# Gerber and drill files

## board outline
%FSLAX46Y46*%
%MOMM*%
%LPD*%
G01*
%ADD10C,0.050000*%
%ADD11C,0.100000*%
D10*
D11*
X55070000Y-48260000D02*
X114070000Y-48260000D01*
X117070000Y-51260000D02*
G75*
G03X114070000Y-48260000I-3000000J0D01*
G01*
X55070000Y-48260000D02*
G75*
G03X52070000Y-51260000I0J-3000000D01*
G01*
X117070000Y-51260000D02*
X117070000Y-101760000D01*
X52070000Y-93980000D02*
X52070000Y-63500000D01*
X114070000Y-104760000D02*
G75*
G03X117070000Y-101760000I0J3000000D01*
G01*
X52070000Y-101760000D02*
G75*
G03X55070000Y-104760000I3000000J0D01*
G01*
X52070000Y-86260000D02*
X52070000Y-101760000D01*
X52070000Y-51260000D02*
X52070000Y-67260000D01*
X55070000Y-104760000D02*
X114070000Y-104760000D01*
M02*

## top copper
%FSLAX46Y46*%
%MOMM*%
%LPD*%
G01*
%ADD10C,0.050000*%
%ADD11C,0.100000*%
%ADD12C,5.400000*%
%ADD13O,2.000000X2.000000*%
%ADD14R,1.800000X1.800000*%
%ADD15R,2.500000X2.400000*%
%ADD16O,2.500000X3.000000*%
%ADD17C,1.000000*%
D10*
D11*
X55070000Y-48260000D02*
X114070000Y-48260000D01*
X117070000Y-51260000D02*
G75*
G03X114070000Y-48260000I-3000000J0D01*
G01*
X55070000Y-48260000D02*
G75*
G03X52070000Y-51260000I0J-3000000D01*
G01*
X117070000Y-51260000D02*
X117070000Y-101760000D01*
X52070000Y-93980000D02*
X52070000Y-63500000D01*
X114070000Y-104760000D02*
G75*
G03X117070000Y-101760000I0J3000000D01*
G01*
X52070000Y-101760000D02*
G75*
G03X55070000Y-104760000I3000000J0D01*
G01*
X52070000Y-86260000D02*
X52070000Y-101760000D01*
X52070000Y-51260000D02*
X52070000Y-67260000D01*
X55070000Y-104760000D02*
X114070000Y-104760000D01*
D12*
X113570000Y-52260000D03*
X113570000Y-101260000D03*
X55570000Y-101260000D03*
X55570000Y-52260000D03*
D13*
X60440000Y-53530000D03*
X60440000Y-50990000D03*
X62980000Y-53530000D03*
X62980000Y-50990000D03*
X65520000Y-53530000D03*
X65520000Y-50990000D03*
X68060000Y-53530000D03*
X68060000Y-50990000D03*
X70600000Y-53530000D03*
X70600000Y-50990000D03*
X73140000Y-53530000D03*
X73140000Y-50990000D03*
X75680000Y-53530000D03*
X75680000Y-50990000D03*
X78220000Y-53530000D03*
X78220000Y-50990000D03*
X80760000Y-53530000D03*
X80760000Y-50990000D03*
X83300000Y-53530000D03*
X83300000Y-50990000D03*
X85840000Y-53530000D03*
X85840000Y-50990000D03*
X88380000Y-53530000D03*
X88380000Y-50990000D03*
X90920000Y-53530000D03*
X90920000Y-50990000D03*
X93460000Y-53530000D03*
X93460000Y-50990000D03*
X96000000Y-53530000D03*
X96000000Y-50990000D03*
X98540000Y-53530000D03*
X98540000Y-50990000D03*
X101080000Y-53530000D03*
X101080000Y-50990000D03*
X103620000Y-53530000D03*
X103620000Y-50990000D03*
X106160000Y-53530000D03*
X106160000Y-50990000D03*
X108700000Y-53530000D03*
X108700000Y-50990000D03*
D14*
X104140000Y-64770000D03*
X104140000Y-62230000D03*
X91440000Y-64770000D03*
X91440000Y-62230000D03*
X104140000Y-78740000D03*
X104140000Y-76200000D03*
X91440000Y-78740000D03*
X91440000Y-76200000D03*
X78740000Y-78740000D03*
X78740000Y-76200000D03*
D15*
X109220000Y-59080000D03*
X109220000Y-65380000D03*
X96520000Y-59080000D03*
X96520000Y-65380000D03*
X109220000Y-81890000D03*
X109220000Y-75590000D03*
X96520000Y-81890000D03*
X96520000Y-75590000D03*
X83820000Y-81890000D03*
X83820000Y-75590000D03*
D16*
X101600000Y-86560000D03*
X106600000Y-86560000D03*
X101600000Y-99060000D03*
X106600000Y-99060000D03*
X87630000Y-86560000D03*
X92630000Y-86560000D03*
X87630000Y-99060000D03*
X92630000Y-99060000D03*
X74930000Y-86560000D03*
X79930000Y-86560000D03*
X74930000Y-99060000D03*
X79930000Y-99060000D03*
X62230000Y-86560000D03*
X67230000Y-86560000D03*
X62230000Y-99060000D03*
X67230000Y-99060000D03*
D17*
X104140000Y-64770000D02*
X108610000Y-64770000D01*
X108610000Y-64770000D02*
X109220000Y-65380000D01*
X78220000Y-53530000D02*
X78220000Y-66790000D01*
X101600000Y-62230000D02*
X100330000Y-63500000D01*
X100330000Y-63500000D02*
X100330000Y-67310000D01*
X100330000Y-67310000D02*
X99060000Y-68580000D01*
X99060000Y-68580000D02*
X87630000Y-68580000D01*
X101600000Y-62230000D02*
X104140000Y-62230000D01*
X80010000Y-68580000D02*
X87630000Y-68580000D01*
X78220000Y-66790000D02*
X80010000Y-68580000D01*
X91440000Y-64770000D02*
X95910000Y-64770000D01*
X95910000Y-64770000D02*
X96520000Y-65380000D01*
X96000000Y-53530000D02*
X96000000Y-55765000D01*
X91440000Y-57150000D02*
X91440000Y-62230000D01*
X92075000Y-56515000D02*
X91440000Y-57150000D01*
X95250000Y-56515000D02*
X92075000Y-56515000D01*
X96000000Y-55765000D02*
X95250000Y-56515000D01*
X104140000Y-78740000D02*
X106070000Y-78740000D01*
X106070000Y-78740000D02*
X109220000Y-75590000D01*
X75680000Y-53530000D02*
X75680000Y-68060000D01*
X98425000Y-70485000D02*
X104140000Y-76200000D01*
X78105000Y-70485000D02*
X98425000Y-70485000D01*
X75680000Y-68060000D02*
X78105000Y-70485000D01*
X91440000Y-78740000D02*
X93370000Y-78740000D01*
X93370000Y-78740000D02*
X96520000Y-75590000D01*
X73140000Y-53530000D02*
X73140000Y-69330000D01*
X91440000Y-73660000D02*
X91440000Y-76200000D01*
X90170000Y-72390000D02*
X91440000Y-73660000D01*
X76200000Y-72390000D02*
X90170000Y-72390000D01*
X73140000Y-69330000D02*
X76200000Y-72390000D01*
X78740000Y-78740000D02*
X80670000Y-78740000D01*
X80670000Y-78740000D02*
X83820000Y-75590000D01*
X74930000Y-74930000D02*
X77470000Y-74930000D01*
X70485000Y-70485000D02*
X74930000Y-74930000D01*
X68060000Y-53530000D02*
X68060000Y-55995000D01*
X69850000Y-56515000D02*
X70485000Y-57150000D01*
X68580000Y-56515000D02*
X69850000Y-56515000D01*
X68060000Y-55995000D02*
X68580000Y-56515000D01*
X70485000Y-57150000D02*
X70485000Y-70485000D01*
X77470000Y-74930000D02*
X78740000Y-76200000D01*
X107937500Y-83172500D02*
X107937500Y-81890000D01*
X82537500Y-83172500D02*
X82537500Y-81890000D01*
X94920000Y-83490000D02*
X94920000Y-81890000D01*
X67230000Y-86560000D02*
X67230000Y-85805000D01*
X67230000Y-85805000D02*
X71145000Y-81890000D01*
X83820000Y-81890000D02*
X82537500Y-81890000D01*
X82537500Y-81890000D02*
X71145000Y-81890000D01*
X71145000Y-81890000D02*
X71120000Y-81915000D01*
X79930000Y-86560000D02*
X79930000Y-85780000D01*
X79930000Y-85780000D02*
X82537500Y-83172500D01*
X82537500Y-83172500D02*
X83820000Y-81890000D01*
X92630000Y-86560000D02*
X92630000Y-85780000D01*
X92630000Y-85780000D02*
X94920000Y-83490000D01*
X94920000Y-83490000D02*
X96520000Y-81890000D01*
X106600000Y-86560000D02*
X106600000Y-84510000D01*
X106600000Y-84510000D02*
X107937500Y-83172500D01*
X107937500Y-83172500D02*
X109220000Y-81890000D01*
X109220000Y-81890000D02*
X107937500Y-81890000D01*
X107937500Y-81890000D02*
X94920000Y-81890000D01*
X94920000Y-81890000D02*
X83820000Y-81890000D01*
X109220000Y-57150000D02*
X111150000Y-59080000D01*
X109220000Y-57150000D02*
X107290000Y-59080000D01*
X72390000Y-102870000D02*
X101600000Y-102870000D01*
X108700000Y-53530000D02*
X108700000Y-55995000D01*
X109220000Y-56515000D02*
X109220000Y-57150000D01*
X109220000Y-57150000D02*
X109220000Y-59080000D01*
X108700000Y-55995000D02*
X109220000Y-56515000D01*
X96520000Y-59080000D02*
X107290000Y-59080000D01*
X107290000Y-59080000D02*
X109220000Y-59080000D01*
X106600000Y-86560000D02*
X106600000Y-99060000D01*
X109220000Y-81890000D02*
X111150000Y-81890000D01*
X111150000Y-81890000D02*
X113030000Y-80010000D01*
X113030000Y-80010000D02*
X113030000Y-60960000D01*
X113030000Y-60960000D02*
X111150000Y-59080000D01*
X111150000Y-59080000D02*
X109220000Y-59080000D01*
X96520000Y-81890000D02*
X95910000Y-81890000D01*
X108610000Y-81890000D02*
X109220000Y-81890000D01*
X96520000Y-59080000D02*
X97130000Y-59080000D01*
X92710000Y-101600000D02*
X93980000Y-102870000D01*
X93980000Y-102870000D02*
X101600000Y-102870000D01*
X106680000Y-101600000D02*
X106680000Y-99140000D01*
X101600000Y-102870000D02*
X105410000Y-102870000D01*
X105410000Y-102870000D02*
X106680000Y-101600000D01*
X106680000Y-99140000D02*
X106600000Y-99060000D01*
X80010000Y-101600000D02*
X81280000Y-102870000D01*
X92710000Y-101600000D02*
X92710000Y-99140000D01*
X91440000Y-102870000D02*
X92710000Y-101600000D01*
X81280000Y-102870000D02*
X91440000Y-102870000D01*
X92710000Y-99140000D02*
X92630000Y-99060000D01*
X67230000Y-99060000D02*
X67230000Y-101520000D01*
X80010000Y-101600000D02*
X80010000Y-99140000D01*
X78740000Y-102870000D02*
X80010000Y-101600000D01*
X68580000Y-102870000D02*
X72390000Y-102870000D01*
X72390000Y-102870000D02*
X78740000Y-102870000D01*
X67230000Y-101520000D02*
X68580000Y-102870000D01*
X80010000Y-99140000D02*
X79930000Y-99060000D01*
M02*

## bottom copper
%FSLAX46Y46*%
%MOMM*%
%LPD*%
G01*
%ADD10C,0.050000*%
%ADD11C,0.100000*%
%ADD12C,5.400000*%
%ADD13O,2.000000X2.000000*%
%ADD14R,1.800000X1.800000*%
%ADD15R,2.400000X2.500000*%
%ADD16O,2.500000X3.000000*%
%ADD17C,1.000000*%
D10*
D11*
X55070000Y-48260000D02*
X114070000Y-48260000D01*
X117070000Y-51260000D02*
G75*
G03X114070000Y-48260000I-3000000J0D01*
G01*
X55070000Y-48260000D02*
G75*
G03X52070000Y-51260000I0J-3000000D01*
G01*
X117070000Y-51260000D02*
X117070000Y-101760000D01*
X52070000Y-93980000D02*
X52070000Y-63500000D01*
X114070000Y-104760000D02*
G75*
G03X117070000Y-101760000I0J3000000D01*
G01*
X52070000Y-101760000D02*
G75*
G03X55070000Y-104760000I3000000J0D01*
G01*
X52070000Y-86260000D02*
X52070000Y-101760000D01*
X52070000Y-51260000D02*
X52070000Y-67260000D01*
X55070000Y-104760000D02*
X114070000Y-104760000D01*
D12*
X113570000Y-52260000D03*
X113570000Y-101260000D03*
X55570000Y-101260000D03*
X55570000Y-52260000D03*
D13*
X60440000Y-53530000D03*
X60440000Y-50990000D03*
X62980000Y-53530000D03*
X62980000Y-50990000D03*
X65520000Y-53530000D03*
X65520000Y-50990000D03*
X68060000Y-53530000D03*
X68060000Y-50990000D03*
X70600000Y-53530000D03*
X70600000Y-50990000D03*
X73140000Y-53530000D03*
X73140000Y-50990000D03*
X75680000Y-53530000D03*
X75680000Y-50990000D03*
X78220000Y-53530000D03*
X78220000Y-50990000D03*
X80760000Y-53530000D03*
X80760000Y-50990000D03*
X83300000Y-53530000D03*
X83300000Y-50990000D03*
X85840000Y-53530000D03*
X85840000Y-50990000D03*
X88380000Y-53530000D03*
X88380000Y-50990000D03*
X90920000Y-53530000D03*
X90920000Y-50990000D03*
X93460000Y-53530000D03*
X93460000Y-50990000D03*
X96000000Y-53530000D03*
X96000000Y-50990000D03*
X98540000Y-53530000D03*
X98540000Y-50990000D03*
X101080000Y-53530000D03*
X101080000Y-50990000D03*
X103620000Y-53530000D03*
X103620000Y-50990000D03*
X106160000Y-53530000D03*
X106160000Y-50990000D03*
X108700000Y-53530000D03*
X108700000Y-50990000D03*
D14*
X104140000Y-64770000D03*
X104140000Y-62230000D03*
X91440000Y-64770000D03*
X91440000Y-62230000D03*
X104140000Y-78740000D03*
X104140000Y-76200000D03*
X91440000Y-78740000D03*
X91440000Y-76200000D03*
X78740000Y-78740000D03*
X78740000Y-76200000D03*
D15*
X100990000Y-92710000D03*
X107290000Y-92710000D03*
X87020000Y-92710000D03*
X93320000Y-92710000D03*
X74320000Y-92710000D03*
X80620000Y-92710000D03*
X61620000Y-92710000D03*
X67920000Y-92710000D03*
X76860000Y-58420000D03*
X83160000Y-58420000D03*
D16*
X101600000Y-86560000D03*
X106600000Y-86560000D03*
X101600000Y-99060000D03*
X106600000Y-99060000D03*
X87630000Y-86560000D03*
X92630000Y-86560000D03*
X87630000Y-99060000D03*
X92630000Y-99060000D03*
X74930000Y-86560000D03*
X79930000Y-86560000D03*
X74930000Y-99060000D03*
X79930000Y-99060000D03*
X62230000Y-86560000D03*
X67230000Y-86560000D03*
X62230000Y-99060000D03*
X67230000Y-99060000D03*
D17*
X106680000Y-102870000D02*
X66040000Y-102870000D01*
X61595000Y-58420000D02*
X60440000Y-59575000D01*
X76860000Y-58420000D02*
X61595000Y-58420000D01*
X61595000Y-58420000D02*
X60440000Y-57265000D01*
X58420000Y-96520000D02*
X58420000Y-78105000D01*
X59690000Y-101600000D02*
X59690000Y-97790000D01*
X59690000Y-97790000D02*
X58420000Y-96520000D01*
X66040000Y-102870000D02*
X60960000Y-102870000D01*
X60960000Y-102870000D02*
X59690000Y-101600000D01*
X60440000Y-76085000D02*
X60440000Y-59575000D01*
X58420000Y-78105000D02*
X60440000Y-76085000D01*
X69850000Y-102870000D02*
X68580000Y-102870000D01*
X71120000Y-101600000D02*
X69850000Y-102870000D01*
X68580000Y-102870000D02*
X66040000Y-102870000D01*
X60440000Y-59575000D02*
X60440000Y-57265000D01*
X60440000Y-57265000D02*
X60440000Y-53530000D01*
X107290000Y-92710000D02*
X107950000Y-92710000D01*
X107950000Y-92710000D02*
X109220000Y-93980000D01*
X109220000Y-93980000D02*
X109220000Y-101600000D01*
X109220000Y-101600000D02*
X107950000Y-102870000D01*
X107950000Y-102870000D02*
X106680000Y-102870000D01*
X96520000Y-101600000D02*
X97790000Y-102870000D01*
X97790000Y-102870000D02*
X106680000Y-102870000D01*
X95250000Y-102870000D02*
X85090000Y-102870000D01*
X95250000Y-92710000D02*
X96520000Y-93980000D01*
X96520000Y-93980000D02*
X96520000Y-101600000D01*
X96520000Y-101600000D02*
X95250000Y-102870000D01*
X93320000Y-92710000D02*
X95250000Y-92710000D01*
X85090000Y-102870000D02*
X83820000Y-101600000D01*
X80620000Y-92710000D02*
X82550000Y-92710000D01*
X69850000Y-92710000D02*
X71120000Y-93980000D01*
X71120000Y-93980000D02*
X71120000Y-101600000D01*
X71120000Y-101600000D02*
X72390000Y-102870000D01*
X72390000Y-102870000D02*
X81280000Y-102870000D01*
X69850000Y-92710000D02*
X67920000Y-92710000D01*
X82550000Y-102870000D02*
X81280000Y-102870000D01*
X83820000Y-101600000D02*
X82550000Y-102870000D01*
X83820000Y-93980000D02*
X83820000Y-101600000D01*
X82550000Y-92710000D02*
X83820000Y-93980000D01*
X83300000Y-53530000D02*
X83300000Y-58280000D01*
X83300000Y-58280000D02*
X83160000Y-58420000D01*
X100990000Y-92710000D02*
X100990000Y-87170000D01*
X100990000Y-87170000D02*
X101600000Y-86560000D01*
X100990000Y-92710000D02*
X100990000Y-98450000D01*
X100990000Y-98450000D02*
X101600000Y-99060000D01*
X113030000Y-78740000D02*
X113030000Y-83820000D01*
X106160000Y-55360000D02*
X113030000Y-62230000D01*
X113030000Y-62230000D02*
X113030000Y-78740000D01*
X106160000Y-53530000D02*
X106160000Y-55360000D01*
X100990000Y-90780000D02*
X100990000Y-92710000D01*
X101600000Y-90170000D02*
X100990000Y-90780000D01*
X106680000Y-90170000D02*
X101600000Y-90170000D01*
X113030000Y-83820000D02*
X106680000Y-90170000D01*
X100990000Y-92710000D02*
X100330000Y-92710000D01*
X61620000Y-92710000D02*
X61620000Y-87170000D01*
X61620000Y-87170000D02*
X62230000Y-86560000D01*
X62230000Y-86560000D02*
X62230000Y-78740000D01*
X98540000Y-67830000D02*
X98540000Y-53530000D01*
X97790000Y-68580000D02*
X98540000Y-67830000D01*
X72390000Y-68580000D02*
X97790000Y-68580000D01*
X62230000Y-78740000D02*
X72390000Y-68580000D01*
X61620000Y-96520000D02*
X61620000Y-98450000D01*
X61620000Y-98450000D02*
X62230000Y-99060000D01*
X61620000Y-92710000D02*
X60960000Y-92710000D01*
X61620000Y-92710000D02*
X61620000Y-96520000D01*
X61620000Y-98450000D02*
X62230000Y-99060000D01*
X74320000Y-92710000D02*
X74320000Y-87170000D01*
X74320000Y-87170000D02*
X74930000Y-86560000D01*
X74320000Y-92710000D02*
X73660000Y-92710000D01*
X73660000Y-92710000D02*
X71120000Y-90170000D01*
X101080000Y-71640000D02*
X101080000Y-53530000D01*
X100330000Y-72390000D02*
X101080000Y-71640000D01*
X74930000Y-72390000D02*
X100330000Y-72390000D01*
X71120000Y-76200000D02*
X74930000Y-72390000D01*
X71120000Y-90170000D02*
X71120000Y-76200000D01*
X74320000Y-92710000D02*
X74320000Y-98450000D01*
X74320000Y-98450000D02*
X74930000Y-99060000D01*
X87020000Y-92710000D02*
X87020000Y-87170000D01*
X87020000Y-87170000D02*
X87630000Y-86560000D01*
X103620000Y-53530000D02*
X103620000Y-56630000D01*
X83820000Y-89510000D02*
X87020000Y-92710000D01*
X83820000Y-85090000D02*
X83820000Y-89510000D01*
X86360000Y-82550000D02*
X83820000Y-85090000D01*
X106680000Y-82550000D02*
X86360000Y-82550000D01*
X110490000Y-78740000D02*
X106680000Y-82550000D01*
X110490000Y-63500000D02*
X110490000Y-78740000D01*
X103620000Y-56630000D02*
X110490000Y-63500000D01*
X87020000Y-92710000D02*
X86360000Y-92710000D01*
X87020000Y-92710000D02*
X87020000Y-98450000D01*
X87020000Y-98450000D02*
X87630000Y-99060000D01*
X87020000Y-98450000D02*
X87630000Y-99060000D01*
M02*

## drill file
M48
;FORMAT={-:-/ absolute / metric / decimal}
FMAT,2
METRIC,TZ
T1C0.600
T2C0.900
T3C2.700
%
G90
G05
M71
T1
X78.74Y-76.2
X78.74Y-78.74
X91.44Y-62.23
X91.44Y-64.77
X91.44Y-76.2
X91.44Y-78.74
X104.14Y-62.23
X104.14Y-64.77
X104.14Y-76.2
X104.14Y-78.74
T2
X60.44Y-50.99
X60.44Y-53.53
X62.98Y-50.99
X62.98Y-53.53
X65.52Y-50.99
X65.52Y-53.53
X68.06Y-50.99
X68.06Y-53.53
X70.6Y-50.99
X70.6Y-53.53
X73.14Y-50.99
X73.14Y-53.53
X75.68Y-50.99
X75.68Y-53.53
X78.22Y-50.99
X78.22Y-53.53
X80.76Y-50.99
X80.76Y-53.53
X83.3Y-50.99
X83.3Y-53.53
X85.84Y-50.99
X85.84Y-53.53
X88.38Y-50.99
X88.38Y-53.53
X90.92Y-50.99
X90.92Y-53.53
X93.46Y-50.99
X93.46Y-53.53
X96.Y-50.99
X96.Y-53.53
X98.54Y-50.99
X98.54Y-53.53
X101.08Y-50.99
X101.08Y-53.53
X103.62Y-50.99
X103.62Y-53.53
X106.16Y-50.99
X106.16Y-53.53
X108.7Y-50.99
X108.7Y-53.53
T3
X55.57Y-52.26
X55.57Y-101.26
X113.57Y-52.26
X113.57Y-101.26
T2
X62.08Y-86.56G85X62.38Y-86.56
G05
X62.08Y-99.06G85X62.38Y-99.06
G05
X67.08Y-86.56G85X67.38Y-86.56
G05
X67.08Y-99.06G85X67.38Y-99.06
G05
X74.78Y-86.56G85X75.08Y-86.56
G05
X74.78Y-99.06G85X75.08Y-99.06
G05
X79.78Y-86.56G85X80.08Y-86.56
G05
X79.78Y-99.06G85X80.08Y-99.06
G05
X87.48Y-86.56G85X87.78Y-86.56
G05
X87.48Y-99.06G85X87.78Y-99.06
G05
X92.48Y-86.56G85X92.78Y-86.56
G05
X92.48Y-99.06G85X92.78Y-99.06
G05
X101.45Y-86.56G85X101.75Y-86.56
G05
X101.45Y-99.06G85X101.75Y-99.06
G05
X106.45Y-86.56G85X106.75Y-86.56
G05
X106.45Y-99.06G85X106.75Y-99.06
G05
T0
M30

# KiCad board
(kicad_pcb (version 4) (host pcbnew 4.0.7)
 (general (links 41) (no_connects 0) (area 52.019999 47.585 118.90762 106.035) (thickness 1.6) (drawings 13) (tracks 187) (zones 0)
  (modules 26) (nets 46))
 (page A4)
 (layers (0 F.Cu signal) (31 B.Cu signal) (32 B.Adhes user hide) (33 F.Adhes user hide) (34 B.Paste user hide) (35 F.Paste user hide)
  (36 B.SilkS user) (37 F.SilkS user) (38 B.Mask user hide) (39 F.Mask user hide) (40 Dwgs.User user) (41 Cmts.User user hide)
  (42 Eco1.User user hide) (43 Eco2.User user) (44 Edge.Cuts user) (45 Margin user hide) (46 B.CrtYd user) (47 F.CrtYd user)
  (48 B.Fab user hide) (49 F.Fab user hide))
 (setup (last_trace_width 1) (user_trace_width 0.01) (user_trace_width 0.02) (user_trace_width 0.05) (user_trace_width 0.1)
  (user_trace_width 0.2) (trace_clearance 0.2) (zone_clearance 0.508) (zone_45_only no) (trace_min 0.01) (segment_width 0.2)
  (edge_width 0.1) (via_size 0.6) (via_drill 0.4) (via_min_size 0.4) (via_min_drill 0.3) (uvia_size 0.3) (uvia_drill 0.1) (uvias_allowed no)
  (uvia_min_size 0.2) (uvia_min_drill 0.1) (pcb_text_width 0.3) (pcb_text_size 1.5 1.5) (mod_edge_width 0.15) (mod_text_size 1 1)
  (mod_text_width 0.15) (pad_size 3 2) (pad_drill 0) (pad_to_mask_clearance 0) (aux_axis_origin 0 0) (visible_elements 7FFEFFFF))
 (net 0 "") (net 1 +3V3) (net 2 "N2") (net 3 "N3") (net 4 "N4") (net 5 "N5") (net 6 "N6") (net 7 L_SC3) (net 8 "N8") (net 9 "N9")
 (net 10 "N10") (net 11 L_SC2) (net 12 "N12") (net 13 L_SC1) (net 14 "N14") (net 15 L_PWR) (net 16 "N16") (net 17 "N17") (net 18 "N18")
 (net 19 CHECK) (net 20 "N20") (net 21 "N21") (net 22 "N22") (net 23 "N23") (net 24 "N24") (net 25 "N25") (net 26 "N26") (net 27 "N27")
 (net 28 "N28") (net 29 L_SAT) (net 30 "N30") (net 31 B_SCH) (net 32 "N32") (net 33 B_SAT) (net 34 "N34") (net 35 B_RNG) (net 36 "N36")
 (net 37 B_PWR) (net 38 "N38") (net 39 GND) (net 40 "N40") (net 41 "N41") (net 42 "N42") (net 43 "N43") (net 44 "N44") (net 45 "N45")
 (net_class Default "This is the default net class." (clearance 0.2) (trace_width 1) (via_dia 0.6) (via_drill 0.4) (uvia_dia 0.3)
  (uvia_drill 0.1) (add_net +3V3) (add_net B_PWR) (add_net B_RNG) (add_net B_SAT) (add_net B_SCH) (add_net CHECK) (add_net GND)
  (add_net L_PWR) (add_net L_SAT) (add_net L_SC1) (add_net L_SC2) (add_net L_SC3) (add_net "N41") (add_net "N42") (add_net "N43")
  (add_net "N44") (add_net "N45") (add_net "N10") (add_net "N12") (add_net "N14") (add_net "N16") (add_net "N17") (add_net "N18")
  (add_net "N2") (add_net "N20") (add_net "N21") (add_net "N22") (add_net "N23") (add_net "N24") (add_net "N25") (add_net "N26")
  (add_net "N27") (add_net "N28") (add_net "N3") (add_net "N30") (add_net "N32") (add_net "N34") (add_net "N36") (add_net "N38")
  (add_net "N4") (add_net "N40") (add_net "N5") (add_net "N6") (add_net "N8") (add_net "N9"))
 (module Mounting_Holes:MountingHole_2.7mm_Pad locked (layer F.Cu) (at 113.57 52.26)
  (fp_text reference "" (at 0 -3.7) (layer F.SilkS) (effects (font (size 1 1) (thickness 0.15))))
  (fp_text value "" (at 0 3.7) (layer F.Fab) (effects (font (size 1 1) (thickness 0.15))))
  (pad 1 thru_hole circle (at 0 0) (size 5.4 5.4) (drill 2.7) (layers *.Cu *.Mask)))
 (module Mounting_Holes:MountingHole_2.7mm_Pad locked (layer F.Cu) (at 113.57 101.26)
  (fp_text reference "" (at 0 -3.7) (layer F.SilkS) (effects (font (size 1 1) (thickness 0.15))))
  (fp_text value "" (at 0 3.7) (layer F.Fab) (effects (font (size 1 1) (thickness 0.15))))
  (pad 1 thru_hole circle (at 0 0) (size 5.4 5.4) (drill 2.7) (layers *.Cu *.Mask)))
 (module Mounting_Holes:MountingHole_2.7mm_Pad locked (layer F.Cu) (at 55.57 101.26)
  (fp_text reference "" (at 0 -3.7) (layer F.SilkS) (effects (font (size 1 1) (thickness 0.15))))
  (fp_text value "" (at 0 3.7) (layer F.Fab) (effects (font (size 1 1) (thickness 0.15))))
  (pad 1 thru_hole circle (at 0 0) (size 5.4 5.4) (drill 2.7) (layers *.Cu *.Mask)))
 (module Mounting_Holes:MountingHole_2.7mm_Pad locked (layer F.Cu) (at 55.57 52.26)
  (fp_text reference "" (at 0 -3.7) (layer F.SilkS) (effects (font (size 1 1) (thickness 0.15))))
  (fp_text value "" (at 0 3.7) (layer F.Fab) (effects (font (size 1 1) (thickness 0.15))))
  (pad 1 thru_hole circle (at 0 0) (size 5.4 5.4) (drill 2.7) (layers *.Cu *.Mask)))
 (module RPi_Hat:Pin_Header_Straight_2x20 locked (layer F.Cu) (at 84.57 52.26 90)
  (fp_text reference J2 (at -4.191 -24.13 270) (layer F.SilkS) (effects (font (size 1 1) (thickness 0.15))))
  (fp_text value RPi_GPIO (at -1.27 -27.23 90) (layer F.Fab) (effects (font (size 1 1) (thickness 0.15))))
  (pad 1 thru_hole oval (at -1.27 -24.13 90) (size 2 2) (drill 0.9) (layers *.Cu *.Mask F.SilkS) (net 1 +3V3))
  (pad 2 thru_hole oval (at 1.27 -24.13 90) (size 2 2) (drill 0.9) (layers *.Cu *.Mask F.SilkS) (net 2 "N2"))
  (pad 3 thru_hole oval (at -1.27 -21.59 90) (size 2 2) (drill 0.9) (layers *.Cu *.Mask F.SilkS) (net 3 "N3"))
  (pad 4 thru_hole oval (at 1.27 -21.59 90) (size 2 2) (drill 0.9) (layers *.Cu *.Mask F.SilkS) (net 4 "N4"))
  (pad 5 thru_hole oval (at -1.27 -19.05 90) (size 2 2) (drill 0.9) (layers *.Cu *.Mask F.SilkS) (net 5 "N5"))
  (pad 6 thru_hole oval (at 1.27 -19.05 90) (size 2 2) (drill 0.9) (layers *.Cu *.Mask F.SilkS) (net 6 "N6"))
  (pad 7 thru_hole oval (at -1.27 -16.51 90) (size 2 2) (drill 0.9) (layers *.Cu *.Mask F.SilkS) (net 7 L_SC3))
  (pad 8 thru_hole oval (at 1.27 -16.51 90) (size 2 2) (drill 0.9) (layers *.Cu *.Mask F.SilkS) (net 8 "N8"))
  (pad 9 thru_hole oval (at -1.27 -13.97 90) (size 2 2) (drill 0.9) (layers *.Cu *.Mask F.SilkS) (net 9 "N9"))
  (pad 10 thru_hole oval (at 1.27 -13.97 90) (size 2 2) (drill 0.9) (layers *.Cu *.Mask F.SilkS) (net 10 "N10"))
  (pad 11 thru_hole oval (at -1.27 -11.43 90) (size 2 2) (drill 0.9) (layers *.Cu *.Mask F.SilkS) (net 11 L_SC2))
  (pad 12 thru_hole oval (at 1.27 -11.43 90) (size 2 2) (drill 0.9) (layers *.Cu *.Mask F.SilkS) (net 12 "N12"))
  (pad 13 thru_hole oval (at -1.27 -8.89 90) (size 2 2) (drill 0.9) (layers *.Cu *.Mask F.SilkS) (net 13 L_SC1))
  (pad 14 thru_hole oval (at 1.27 -8.89 90) (size 2 2) (drill 0.9) (layers *.Cu *.Mask F.SilkS) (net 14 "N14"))
  (pad 15 thru_hole oval (at -1.27 -6.35 90) (size 2 2) (drill 0.9) (layers *.Cu *.Mask F.SilkS) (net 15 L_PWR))
  (pad 16 thru_hole oval (at 1.27 -6.35 90) (size 2 2) (drill 0.9) (layers *.Cu *.Mask F.SilkS) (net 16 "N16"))
  (pad 17 thru_hole oval (at -1.27 -3.81 90) (size 2 2) (drill 0.9) (layers *.Cu *.Mask F.SilkS) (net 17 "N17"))
  (pad 18 thru_hole oval (at 1.27 -3.81 90) (size 2 2) (drill 0.9) (layers *.Cu *.Mask F.SilkS) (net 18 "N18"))
  (pad 19 thru_hole oval (at -1.27 -1.27 90) (size 2 2) (drill 0.9) (layers *.Cu *.Mask F.SilkS) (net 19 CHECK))
  (pad 20 thru_hole oval (at 1.27 -1.27 90) (size 2 2) (drill 0.9) (layers *.Cu *.Mask F.SilkS) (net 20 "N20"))
  (pad 21 thru_hole oval (at -1.27 1.27 90) (size 2 2) (drill 0.9) (layers *.Cu *.Mask F.SilkS) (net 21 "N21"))
  (pad 22 thru_hole oval (at 1.27 1.27 90) (size 2 2) (drill 0.9) (layers *.Cu *.Mask F.SilkS) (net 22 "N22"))
  (pad 23 thru_hole oval (at -1.27 3.81 90) (size 2 2) (drill 0.9) (layers *.Cu *.Mask F.SilkS) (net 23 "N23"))
  (pad 24 thru_hole oval (at 1.27 3.81 90) (size 2 2) (drill 0.9) (layers *.Cu *.Mask F.SilkS) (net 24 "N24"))
  (pad 25 thru_hole oval (at -1.27 6.35 90) (size 2 2) (drill 0.9) (layers *.Cu *.Mask F.SilkS) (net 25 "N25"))
  (pad 26 thru_hole oval (at 1.27 6.35 90) (size 2 2) (drill 0.9) (layers *.Cu *.Mask F.SilkS) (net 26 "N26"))
  (pad 27 thru_hole oval (at -1.27 8.89 90) (size 2 2) (drill 0.9) (layers *.Cu *.Mask F.SilkS) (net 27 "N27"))
  (pad 28 thru_hole oval (at 1.27 8.89 90) (size 2 2) (drill 0.9) (layers *.Cu *.Mask F.SilkS) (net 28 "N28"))
  (pad 29 thru_hole oval (at -1.27 11.43 90) (size 2 2) (drill 0.9) (layers *.Cu *.Mask F.SilkS) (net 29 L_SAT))
  (pad 30 thru_hole oval (at 1.27 11.43 90) (size 2 2) (drill 0.9) (layers *.Cu *.Mask F.SilkS) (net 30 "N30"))
  (pad 31 thru_hole oval (at -1.27 13.97 90) (size 2 2) (drill 0.9) (layers *.Cu *.Mask F.SilkS) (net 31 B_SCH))
  (pad 32 thru_hole oval (at 1.27 13.97 90) (size 2 2) (drill 0.9) (layers *.Cu *.Mask F.SilkS) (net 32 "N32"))
  (pad 33 thru_hole oval (at -1.27 16.51 90) (size 2 2) (drill 0.9) (layers *.Cu *.Mask F.SilkS) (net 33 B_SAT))
  (pad 34 thru_hole oval (at 1.27 16.51 90) (size 2 2) (drill 0.9) (layers *.Cu *.Mask F.SilkS) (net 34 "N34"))
  (pad 35 thru_hole oval (at -1.27 19.05 90) (size 2 2) (drill 0.9) (layers *.Cu *.Mask F.SilkS) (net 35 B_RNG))
  (pad 36 thru_hole oval (at 1.27 19.05 90) (size 2 2) (drill 0.9) (layers *.Cu *.Mask F.SilkS) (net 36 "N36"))
  (pad 37 thru_hole oval (at -1.27 21.59 90) (size 2 2) (drill 0.9) (layers *.Cu *.Mask F.SilkS) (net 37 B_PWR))
  (pad 38 thru_hole oval (at 1.27 21.59 90) (size 2 2) (drill 0.9) (layers *.Cu *.Mask F.SilkS) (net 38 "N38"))
  (pad 39 thru_hole oval (at -1.27 24.13 90) (size 2 2) (drill 0.9) (layers *.Cu *.Mask F.SilkS) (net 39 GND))
  (pad 40 thru_hole oval (at 1.27 24.13 90) (size 2 2) (drill 0.9) (layers *.Cu *.Mask F.SilkS) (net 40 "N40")))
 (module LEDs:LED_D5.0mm (layer F.Cu) (at 104.14 64.77 90)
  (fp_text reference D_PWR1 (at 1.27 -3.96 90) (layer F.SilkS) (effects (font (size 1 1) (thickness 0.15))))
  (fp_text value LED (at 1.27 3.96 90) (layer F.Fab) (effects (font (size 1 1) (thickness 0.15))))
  (pad 1 thru_hole rect (at 0 0 90) (size 1.8 1.8) (drill 0.6) (layers *.Cu *.Mask) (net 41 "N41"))
  (pad 2 thru_hole rect (at 2.54 0 90) (size 1.8 1.8) (drill 0.6) (layers *.Cu *.Mask) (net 15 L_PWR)))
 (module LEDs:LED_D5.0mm (layer F.Cu) (at 91.44 64.77 90)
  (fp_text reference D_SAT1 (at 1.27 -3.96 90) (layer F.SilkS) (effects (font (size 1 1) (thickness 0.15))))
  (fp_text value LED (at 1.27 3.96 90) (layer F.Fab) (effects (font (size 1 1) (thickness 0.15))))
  (pad 1 thru_hole rect (at 0 0 90) (size 1.8 1.8) (drill 0.6) (layers *.Cu *.Mask) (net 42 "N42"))
  (pad 2 thru_hole rect (at 2.54 0 90) (size 1.8 1.8) (drill 0.6) (layers *.Cu *.Mask) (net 29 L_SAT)))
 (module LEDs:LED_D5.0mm (layer F.Cu) (at 104.14 78.74 90)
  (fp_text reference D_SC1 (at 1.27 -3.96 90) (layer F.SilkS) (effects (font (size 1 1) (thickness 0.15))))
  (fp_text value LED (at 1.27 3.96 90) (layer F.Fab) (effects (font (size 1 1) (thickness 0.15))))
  (pad 1 thru_hole rect (at 0 0 90) (size 1.8 1.8) (drill 0.6) (layers *.Cu *.Mask) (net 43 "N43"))
  (pad 2 thru_hole rect (at 2.54 0 90) (size 1.8 1.8) (drill 0.6) (layers *.Cu *.Mask) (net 13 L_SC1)))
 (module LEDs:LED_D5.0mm (layer F.Cu) (at 91.44 78.74 90)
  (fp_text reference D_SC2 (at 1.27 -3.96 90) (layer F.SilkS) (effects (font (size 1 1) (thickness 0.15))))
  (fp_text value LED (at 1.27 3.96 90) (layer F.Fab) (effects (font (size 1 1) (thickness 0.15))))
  (pad 1 thru_hole rect (at 0 0 90) (size 1.8 1.8) (drill 0.6) (layers *.Cu *.Mask) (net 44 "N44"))
  (pad 2 thru_hole rect (at 2.54 0 90) (size 1.8 1.8) (drill 0.6) (layers *.Cu *.Mask) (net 11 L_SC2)))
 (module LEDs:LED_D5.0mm (layer F.Cu) (at 78.74 78.74 90)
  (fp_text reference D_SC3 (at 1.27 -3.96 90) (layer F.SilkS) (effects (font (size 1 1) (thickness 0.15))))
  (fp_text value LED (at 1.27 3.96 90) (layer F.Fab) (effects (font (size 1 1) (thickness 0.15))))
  (pad 1 thru_hole rect (at 0 0 90) (size 1.8 1.8) (drill 0.6) (layers *.Cu *.Mask) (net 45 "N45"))
  (pad 2 thru_hole rect (at 2.54 0 90) (size 1.8 1.8) (drill 0.6) (layers *.Cu *.Mask) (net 7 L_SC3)))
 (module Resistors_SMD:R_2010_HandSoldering (layer B.Cu) (at 104.14 92.71)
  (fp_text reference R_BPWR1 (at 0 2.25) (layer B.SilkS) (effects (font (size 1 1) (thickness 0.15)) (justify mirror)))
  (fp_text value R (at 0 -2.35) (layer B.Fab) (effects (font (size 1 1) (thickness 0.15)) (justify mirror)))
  (pad 1 smd rect (at -3.15 0) (size 2.4 2.5) (layers B.Cu B.Paste B.Mask) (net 37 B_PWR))
  (pad 2 smd rect (at 3.15 0) (size 2.4 2.5) (layers B.Cu B.Paste B.Mask) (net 1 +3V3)))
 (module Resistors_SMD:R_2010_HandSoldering (layer B.Cu) (at 90.17 92.71)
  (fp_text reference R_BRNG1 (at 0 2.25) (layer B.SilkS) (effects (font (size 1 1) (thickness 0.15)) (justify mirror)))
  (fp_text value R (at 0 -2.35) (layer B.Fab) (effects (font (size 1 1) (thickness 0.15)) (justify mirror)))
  (pad 1 smd rect (at -3.15 0) (size 2.4 2.5) (layers B.Cu B.Paste B.Mask) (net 35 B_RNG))
  (pad 2 smd rect (at 3.15 0) (size 2.4 2.5) (layers B.Cu B.Paste B.Mask) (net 1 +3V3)))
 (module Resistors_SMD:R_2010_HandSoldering (layer B.Cu) (at 77.47 92.71)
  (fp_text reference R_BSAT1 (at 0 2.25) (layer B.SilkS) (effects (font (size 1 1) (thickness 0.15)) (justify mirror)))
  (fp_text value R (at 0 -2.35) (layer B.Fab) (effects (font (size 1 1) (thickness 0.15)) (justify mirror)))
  (pad 1 smd rect (at -3.15 0) (size 2.4 2.5) (layers B.Cu B.Paste B.Mask) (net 33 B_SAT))
  (pad 2 smd rect (at 3.15 0) (size 2.4 2.5) (layers B.Cu B.Paste B.Mask) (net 1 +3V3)))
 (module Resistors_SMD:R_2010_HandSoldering (layer B.Cu) (at 64.77 92.71)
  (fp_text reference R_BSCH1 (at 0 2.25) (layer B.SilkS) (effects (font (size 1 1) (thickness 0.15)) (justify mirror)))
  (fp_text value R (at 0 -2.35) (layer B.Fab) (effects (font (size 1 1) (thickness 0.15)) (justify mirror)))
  (pad 1 smd rect (at -3.15 0) (size 2.4 2.5) (layers B.Cu B.Paste B.Mask) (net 31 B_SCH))
  (pad 2 smd rect (at 3.15 0) (size 2.4 2.5) (layers B.Cu B.Paste B.Mask) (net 1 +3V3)))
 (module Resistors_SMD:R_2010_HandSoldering (layer B.Cu) (at 80.01 58.42)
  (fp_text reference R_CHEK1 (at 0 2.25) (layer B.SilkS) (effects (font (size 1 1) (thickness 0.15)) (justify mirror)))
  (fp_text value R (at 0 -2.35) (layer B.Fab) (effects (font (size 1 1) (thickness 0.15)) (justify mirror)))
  (pad 1 smd rect (at -3.15 0) (size 2.4 2.5) (layers B.Cu B.Paste B.Mask) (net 1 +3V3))
  (pad 2 smd rect (at 3.15 0) (size 2.4 2.5) (layers B.Cu B.Paste B.Mask) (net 19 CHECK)))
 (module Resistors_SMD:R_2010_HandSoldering (layer F.Cu) (at 109.22 62.23 270)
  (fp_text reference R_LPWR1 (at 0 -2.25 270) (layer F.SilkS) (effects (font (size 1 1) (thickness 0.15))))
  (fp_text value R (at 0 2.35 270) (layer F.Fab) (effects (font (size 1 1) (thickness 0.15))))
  (pad 1 smd rect (at -3.15 0 270) (size 2.4 2.5) (layers F.Cu F.Paste F.Mask) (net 39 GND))
  (pad 2 smd rect (at 3.15 0 270) (size 2.4 2.5) (layers F.Cu F.Paste F.Mask) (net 41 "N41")))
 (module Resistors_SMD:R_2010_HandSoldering (layer F.Cu) (at 96.52 62.23 270)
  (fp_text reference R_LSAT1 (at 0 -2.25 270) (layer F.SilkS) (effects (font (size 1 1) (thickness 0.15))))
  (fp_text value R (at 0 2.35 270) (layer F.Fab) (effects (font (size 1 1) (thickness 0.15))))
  (pad 1 smd rect (at -3.15 0 270) (size 2.4 2.5) (layers F.Cu F.Paste F.Mask) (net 39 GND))
  (pad 2 smd rect (at 3.15 0 270) (size 2.4 2.5) (layers F.Cu F.Paste F.Mask) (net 42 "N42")))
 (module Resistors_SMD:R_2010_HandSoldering (layer F.Cu) (at 109.22 78.74 90)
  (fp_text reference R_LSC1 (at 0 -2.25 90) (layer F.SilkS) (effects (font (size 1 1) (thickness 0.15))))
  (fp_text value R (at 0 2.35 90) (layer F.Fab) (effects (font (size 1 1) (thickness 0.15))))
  (pad 1 smd rect (at -3.15 0 90) (size 2.4 2.5) (layers F.Cu F.Paste F.Mask) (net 39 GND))
  (pad 2 smd rect (at 3.15 0 90) (size 2.4 2.5) (layers F.Cu F.Paste F.Mask) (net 43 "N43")))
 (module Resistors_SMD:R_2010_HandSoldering (layer F.Cu) (at 96.52 78.74 90)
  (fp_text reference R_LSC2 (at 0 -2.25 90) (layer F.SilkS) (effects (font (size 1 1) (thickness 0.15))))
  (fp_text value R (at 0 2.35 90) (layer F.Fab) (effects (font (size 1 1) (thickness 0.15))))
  (pad 1 smd rect (at -3.15 0 90) (size 2.4 2.5) (layers F.Cu F.Paste F.Mask) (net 39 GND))
  (pad 2 smd rect (at 3.15 0 90) (size 2.4 2.5) (layers F.Cu F.Paste F.Mask) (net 44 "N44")))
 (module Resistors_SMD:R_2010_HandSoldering (layer F.Cu) (at 83.82 78.74 90)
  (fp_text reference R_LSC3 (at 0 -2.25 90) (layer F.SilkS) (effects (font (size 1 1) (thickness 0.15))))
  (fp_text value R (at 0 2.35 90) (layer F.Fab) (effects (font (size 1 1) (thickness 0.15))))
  (pad 1 smd rect (at -3.15 0 90) (size 2.4 2.5) (layers F.Cu F.Paste F.Mask) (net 39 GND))
  (pad 2 smd rect (at 3.15 0 90) (size 2.4 2.5) (layers F.Cu F.Paste F.Mask) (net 45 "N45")))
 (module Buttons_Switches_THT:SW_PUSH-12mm (layer F.Cu) (at 101.6 99.06 90)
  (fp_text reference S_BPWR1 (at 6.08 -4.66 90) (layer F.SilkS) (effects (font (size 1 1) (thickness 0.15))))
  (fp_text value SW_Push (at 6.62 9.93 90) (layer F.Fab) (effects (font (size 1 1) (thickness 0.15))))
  (pad 1 thru_hole oval (at 12.5 0 90) (size 3 2.5) (drill oval 0.9 1.2) (layers *.Cu *.Mask) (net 37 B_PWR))
  (pad 2 thru_hole oval (at 12.5 5 90) (size 3 2.5) (drill oval 0.9 1.2) (layers *.Cu *.Mask) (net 39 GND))
  (pad 1 thru_hole oval (at 0 0 90) (size 3 2.5) (drill oval 0.9 1.2) (layers *.Cu *.Mask) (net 37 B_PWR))
  (pad 2 thru_hole oval (at 0 5 90) (size 3 2.5) (drill oval 0.9 1.2) (layers *.Cu *.Mask) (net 39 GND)))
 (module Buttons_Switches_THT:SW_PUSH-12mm (layer F.Cu) (at 87.63 99.06 90)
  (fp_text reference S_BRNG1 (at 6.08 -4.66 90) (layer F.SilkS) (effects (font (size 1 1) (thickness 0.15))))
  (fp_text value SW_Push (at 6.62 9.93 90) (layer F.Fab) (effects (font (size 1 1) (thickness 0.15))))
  (pad 1 thru_hole oval (at 12.5 0 90) (size 3 2.5) (drill oval 0.9 1.2) (layers *.Cu *.Mask) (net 35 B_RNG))
  (pad 2 thru_hole oval (at 12.5 5 90) (size 3 2.5) (drill oval 0.9 1.2) (layers *.Cu *.Mask) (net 39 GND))
  (pad 1 thru_hole oval (at 0 0 90) (size 3 2.5) (drill oval 0.9 1.2) (layers *.Cu *.Mask) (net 35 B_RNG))
  (pad 2 thru_hole oval (at 0 5 90) (size 3 2.5) (drill oval 0.9 1.2) (layers *.Cu *.Mask) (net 39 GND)))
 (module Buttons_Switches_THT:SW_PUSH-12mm (layer F.Cu) (at 74.93 99.06 90)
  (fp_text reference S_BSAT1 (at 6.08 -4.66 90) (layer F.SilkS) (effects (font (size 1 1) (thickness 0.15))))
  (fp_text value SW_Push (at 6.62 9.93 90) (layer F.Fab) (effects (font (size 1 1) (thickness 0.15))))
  (pad 1 thru_hole oval (at 12.5 0 90) (size 3 2.5) (drill oval 0.9 1.2) (layers *.Cu *.Mask) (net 33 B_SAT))
  (pad 2 thru_hole oval (at 12.5 5 90) (size 3 2.5) (drill oval 0.9 1.2) (layers *.Cu *.Mask) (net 39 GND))
  (pad 1 thru_hole oval (at 0 0 90) (size 3 2.5) (drill oval 0.9 1.2) (layers *.Cu *.Mask) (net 33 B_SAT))
  (pad 2 thru_hole oval (at 0 5 90) (size 3 2.5) (drill oval 0.9 1.2) (layers *.Cu *.Mask) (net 39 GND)))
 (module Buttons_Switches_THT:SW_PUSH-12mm (layer F.Cu) (at 62.23 99.06 90)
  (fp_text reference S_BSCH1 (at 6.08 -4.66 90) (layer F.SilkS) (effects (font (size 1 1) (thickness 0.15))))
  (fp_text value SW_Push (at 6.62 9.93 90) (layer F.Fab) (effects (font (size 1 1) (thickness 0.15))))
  (pad 1 thru_hole oval (at 12.5 0 90) (size 3 2.5) (drill oval 0.9 1.2) (layers *.Cu *.Mask) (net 31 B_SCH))
  (pad 2 thru_hole oval (at 12.5 5 90) (size 3 2.5) (drill oval 0.9 1.2) (layers *.Cu *.Mask) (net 39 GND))
  (pad 1 thru_hole oval (at 0 0 90) (size 3 2.5) (drill oval 0.9 1.2) (layers *.Cu *.Mask) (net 31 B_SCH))
  (pad 2 thru_hole oval (at 0 5 90) (size 3 2.5) (drill oval 0.9 1.2) (layers *.Cu *.Mask) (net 39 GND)))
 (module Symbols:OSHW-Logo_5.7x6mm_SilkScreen (layer B.Cu) (at 65.6082 63.119 90)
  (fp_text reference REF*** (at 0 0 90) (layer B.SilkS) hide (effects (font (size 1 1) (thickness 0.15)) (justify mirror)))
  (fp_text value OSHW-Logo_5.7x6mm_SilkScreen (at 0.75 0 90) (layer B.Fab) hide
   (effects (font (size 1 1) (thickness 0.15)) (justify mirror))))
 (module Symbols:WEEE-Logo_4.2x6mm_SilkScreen (layer B.Cu) (at 65.16624 69.25564 90)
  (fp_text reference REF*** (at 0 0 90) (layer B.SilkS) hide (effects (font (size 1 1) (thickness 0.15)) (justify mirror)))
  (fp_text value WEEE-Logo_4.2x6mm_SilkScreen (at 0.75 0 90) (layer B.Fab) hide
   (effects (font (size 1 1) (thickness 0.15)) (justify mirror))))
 (gr_line (start 55.07 48.26) (end 114.07 48.26) (angle 90) (layer Edge.Cuts) (width 0.1))
 (gr_arc (start 114.07 51.26) (end 114.07 48.26) (angle 90) (layer Edge.Cuts) (width 0.1))
 (gr_arc (start 55.07 51.26) (end 52.07 51.26) (angle 90) (layer Edge.Cuts) (width 0.1))
 (gr_line (start 117.07 51.26) (end 117.07 101.76) (angle 90) (layer Edge.Cuts) (width 0.1))
 (gr_line (start 52.07 93.98) (end 52.07 63.5) (angle 90) (layer Edge.Cuts) (width 0.1))
 (gr_arc (start 114.07 101.76) (end 117.07 101.76) (angle 90) (layer Edge.Cuts) (width 0.1))
 (gr_arc (start 55.07 101.76) (end 55.07 104.76) (angle 90) (layer Edge.Cuts) (width 0.1))
 (gr_line (start 52.07 86.26) (end 52.07 101.76) (layer Edge.Cuts) (width 0.1))
 (gr_line (start 52.07 51.26) (end 52.07 67.26) (layer Edge.Cuts) (width 0.1))
 (gr_line (start 55.07 104.76) (end 114.07 104.76) (angle 90) (layer Edge.Cuts) (width 0.1))
 (segment (start 104.14 64.77) (end 108.61 64.77) (width 1) (layer F.Cu) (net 41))
 (segment (start 108.61 64.77) (end 109.22 65.38) (width 1) (layer F.Cu) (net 41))
 (segment (start 78.22 53.53) (end 78.22 66.79) (width 1) (layer F.Cu) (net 15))
 (segment (start 101.6 62.23) (end 100.33 63.5) (width 1) (layer F.Cu) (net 15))
 (segment (start 100.33 63.5) (end 100.33 67.31) (width 1) (layer F.Cu) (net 15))
 (segment (start 100.33 67.31) (end 99.06 68.58) (width 1) (layer F.Cu) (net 15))
 (segment (start 99.06 68.58) (end 87.63 68.58) (width 1) (layer F.Cu) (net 15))
 (segment (start 101.6 62.23) (end 104.14 62.23) (width 1) (layer F.Cu) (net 15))
 (segment (start 80.01 68.58) (end 87.63 68.58) (width 1) (layer F.Cu) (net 15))
 (segment (start 78.22 66.79) (end 80.01 68.58) (width 1) (layer F.Cu) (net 15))
 (segment (start 91.44 64.77) (end 95.91 64.77) (width 1) (layer F.Cu) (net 42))
 (segment (start 95.91 64.77) (end 96.52 65.38) (width 1) (layer F.Cu) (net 42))
 (segment (start 96 53.53) (end 96 55.765) (width 1) (layer F.Cu) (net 29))
 (segment (start 91.44 57.15) (end 91.44 62.23) (width 1) (layer F.Cu) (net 29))
 (segment (start 92.075 56.515) (end 91.44 57.15) (width 1) (layer F.Cu) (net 29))
 (segment (start 95.25 56.515) (end 92.075 56.515) (width 1) (layer F.Cu) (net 29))
 (segment (start 96 55.765) (end 95.25 56.515) (width 1) (layer F.Cu) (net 29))
 (segment (start 104.14 78.74) (end 106.07 78.74) (width 1) (layer F.Cu) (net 43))
 (segment (start 106.07 78.74) (end 109.22 75.59) (width 1) (layer F.Cu) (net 43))
 (segment (start 75.68 53.53) (end 75.68 68.06) (width 1) (layer F.Cu) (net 13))
 (segment (start 98.425 70.485) (end 104.14 76.2) (width 1) (layer F.Cu) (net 13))
 (segment (start 78.105 70.485) (end 98.425 70.485) (width 1) (layer F.Cu) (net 13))
 (segment (start 75.68 68.06) (end 78.105 70.485) (width 1) (layer F.Cu) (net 13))
 (segment (start 91.44 78.74) (end 93.37 78.74) (width 1) (layer F.Cu) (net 44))
 (segment (start 93.37 78.74) (end 96.52 75.59) (width 1) (layer F.Cu) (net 44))
 (segment (start 73.14 53.53) (end 73.14 69.33) (width 1) (layer F.Cu) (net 11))
 (segment (start 91.44 73.66) (end 91.44 76.2) (width 1) (layer F.Cu) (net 11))
 (segment (start 90.17 72.39) (end 91.44 73.66) (width 1) (layer F.Cu) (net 11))
 (segment (start 76.2 72.39) (end 90.17 72.39) (width 1) (layer F.Cu) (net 11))
 (segment (start 73.14 69.33) (end 76.2 72.39) (width 1) (layer F.Cu) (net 11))
 (segment (start 78.74 78.74) (end 80.67 78.74) (width 1) (layer F.Cu) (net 45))
 (segment (start 80.67 78.74) (end 83.82 75.59) (width 1) (layer F.Cu) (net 45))
 (segment (start 74.93 74.93) (end 77.47 74.93) (width 1) (layer F.Cu) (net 7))
 (segment (start 70.485 70.485) (end 74.93 74.93) (width 1) (layer F.Cu) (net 7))
 (segment (start 68.06 53.53) (end 68.06 55.995) (width 1) (layer F.Cu) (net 7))
 (segment (start 69.85 56.515) (end 70.485 57.15) (width 1) (layer F.Cu) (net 7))
 (segment (start 68.58 56.515) (end 69.85 56.515) (width 1) (layer F.Cu) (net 7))
 (segment (start 68.06 55.995) (end 68.58 56.515) (width 1) (layer F.Cu) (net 7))
 (segment (start 70.485 57.15) (end 70.485 70.485) (width 1) (layer F.Cu) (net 7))
 (segment (start 77.47 74.93) (end 78.74 76.2) (width 1) (layer F.Cu) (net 7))
 (segment (start 106.68 102.87) (end 66.04 102.87) (width 1) (layer B.Cu) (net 1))
 (segment (start 61.595 58.42) (end 60.44 59.575) (width 1) (layer B.Cu) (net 1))
 (segment (start 76.86 58.42) (end 61.595 58.42) (width 1) (layer B.Cu) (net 1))
 (segment (start 61.595 58.42) (end 60.44 57.265) (width 1) (layer B.Cu) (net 1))
 (segment (start 58.42 96.52) (end 58.42 78.105) (width 1) (layer B.Cu) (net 1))
 (segment (start 59.69 101.6) (end 59.69 97.79) (width 1) (layer B.Cu) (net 1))
 (segment (start 59.69 97.79) (end 58.42 96.52) (width 1) (layer B.Cu) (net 1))
 (segment (start 66.04 102.87) (end 60.96 102.87) (width 1) (layer B.Cu) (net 1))
 (segment (start 60.96 102.87) (end 59.69 101.6) (width 1) (layer B.Cu) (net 1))
 (segment (start 60.44 76.085) (end 60.44 59.575) (width 1) (layer B.Cu) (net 1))
 (segment (start 58.42 78.105) (end 60.44 76.085) (width 1) (layer B.Cu) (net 1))
 (segment (start 69.85 102.87) (end 68.58 102.87) (width 1) (layer B.Cu) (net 1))
 (segment (start 71.12 101.6) (end 69.85 102.87) (width 1) (layer B.Cu) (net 1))
 (segment (start 68.58 102.87) (end 66.04 102.87) (width 1) (layer B.Cu) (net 1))
 (segment (start 60.44 59.575) (end 60.44 57.265) (width 1) (layer B.Cu) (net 1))
 (segment (start 60.44 57.265) (end 60.44 53.53) (width 1) (layer B.Cu) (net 1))
 (segment (start 107.29 92.71) (end 107.95 92.71) (width 1) (layer B.Cu) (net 1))
 (segment (start 107.95 92.71) (end 109.22 93.98) (width 1) (layer B.Cu) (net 1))
 (segment (start 109.22 93.98) (end 109.22 101.6) (width 1) (layer B.Cu) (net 1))
 (segment (start 109.22 101.6) (end 107.95 102.87) (width 1) (layer B.Cu) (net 1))
 (segment (start 107.95 102.87) (end 106.68 102.87) (width 1) (layer B.Cu) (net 1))
 (segment (start 96.52 101.6) (end 97.79 102.87) (width 1) (layer B.Cu) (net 1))
 (segment (start 97.79 102.87) (end 106.68 102.87) (width 1) (layer B.Cu) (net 1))
 (segment (start 95.25 102.87) (end 85.09 102.87) (width 1) (layer B.Cu) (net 1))
 (segment (start 95.25 92.71) (end 96.52 93.98) (width 1) (layer B.Cu) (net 1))
 (segment (start 96.52 93.98) (end 96.52 101.6) (width 1) (layer B.Cu) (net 1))
 (segment (start 96.52 101.6) (end 95.25 102.87) (width 1) (layer B.Cu) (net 1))
 (segment (start 93.32 92.71) (end 95.25 92.71) (width 1) (layer B.Cu) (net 1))
 (segment (start 85.09 102.87) (end 83.82 101.6) (width 1) (layer B.Cu) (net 1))
 (segment (start 80.62 92.71) (end 82.55 92.71) (width 1) (layer B.Cu) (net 1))
 (segment (start 69.85 92.71) (end 71.12 93.98) (width 1) (layer B.Cu) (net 1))
 (segment (start 71.12 93.98) (end 71.12 101.6) (width 1) (layer B.Cu) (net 1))
 (segment (start 71.12 101.6) (end 72.39 102.87) (width 1) (layer B.Cu) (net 1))
 (segment (start 72.39 102.87) (end 81.28 102.87) (width 1) (layer B.Cu) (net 1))
 (segment (start 69.85 92.71) (end 67.92 92.71) (width 1) (layer B.Cu) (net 1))
 (segment (start 82.55 102.87) (end 81.28 102.87) (width 1) (layer B.Cu) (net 1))
 (segment (start 83.82 101.6) (end 82.55 102.87) (width 1) (layer B.Cu) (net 1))
 (segment (start 83.82 93.98) (end 83.82 101.6) (width 1) (layer B.Cu) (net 1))
 (segment (start 82.55 92.71) (end 83.82 93.98) (width 1) (layer B.Cu) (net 1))
 (segment (start 107.9375 83.1725) (end 107.9375 81.89) (width 1) (layer F.Cu) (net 39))
 (segment (start 82.5375 83.1725) (end 82.5375 81.89) (width 1) (layer F.Cu) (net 39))
 (segment (start 94.92 83.49) (end 94.92 81.89) (width 1) (layer F.Cu) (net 39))
 (segment (start 67.23 86.56) (end 67.23 85.805) (width 1) (layer F.Cu) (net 39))
 (segment (start 67.23 85.805) (end 71.145 81.89) (width 1) (layer F.Cu) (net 39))
 (segment (start 83.82 81.89) (end 82.5375 81.89) (width 1) (layer F.Cu) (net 39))
 (segment (start 82.5375 81.89) (end 71.145 81.89) (width 1) (layer F.Cu) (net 39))
 (segment (start 71.145 81.89) (end 71.12 81.915) (width 1) (layer F.Cu) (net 39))
 (segment (start 79.93 86.56) (end 79.93 85.78) (width 1) (layer F.Cu) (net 39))
 (segment (start 79.93 85.78) (end 82.5375 83.1725) (width 1) (layer F.Cu) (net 39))
 (segment (start 82.5375 83.1725) (end 83.82 81.89) (width 1) (layer F.Cu) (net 39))
 (segment (start 92.63 86.56) (end 92.63 85.78) (width 1) (layer F.Cu) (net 39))
 (segment (start 92.63 85.78) (end 94.92 83.49) (width 1) (layer F.Cu) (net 39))
 (segment (start 94.92 83.49) (end 96.52 81.89) (width 1) (layer F.Cu) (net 39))
 (segment (start 106.6 86.56) (end 106.6 84.51) (width 1) (layer F.Cu) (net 39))
 (segment (start 106.6 84.51) (end 107.9375 83.1725) (width 1) (layer F.Cu) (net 39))
 (segment (start 107.9375 83.1725) (end 109.22 81.89) (width 1) (layer F.Cu) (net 39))
 (segment (start 109.22 81.89) (end 107.9375 81.89) (width 1) (layer F.Cu) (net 39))
 (segment (start 107.9375 81.89) (end 94.92 81.89) (width 1) (layer F.Cu) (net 39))
 (segment (start 94.92 81.89) (end 83.82 81.89) (width 1) (layer F.Cu) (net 39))
 (segment (start 109.22 57.15) (end 111.15 59.08) (width 1) (layer F.Cu) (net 39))
 (segment (start 109.22 57.15) (end 107.29 59.08) (width 1) (layer F.Cu) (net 39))
 (segment (start 72.39 102.87) (end 101.6 102.87) (width 1) (layer F.Cu) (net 39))
 (segment (start 108.7 53.53) (end 108.7 55.995) (width 1) (layer F.Cu) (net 39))
 (segment (start 109.22 56.515) (end 109.22 57.15) (width 1) (layer F.Cu) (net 39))
 (segment (start 109.22 57.15) (end 109.22 59.08) (width 1) (layer F.Cu) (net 39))
 (segment (start 108.7 55.995) (end 109.22 56.515) (width 1) (layer F.Cu) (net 39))
 (segment (start 96.52 59.08) (end 107.29 59.08) (width 1) (layer F.Cu) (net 39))
 (segment (start 107.29 59.08) (end 109.22 59.08) (width 1) (layer F.Cu) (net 39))
 (segment (start 106.6 86.56) (end 106.6 99.06) (width 1) (layer F.Cu) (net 39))
 (segment (start 109.22 81.89) (end 111.15 81.89) (width 1) (layer F.Cu) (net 39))
 (segment (start 111.15 81.89) (end 113.03 80.01) (width 1) (layer F.Cu) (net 39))
 (segment (start 113.03 80.01) (end 113.03 60.96) (width 1) (layer F.Cu) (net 39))
 (segment (start 113.03 60.96) (end 111.15 59.08) (width 1) (layer F.Cu) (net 39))
 (segment (start 111.15 59.08) (end 109.22 59.08) (width 1) (layer F.Cu) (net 39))
 (segment (start 96.52 81.89) (end 95.91 81.89) (width 1) (layer F.Cu) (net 39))
 (segment (start 108.61 81.89) (end 109.22 81.89) (width 1) (layer F.Cu) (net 39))
 (segment (start 96.52 59.08) (end 97.13 59.08) (width 1) (layer F.Cu) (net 39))
 (segment (start 92.71 101.6) (end 93.98 102.87) (width 1) (layer F.Cu) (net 39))
 (segment (start 93.98 102.87) (end 101.6 102.87) (width 1) (layer F.Cu) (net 39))
 (segment (start 106.68 101.6) (end 106.68 99.14) (width 1) (layer F.Cu) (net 39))
 (segment (start 101.6 102.87) (end 105.41 102.87) (width 1) (layer F.Cu) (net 39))
 (segment (start 105.41 102.87) (end 106.68 101.6) (width 1) (layer F.Cu) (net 39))
 (segment (start 106.68 99.14) (end 106.6 99.06) (width 1) (layer F.Cu) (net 39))
 (segment (start 80.01 101.6) (end 81.28 102.87) (width 1) (layer F.Cu) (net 39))
 (segment (start 92.71 101.6) (end 92.71 99.14) (width 1) (layer F.Cu) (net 39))
 (segment (start 91.44 102.87) (end 92.71 101.6) (width 1) (layer F.Cu) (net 39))
 (segment (start 81.28 102.87) (end 91.44 102.87) (width 1) (layer F.Cu) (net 39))
 (segment (start 92.71 99.14) (end 92.63 99.06) (width 1) (layer F.Cu) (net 39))
 (segment (start 67.23 99.06) (end 67.23 101.52) (width 1) (layer F.Cu) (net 39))
 (segment (start 80.01 101.6) (end 80.01 99.14) (width 1) (layer F.Cu) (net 39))
 (segment (start 78.74 102.87) (end 80.01 101.6) (width 1) (layer F.Cu) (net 39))
 (segment (start 68.58 102.87) (end 72.39 102.87) (width 1) (layer F.Cu) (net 39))
 (segment (start 72.39 102.87) (end 78.74 102.87) (width 1) (layer F.Cu) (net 39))
 (segment (start 67.23 101.52) (end 68.58 102.87) (width 1) (layer F.Cu) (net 39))
 (segment (start 80.01 99.14) (end 79.93 99.06) (width 1) (layer F.Cu) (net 39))
 (segment (start 83.3 53.53) (end 83.3 58.28) (width 1) (layer B.Cu) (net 19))
 (segment (start 83.3 58.28) (end 83.16 58.42) (width 1) (layer B.Cu) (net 19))
 (segment (start 100.99 92.71) (end 100.99 87.17) (width 1) (layer B.Cu) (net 37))
 (segment (start 100.99 87.17) (end 101.6 86.56) (width 1) (layer B.Cu) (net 37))
 (segment (start 100.99 92.71) (end 100.99 98.45) (width 1) (layer B.Cu) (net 37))
 (segment (start 100.99 98.45) (end 101.6 99.06) (width 1) (layer B.Cu) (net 37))
 (segment (start 113.03 78.74) (end 113.03 83.82) (width 1) (layer B.Cu) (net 37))
 (segment (start 106.16 55.36) (end 113.03 62.23) (width 1) (layer B.Cu) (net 37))
 (segment (start 113.03 62.23) (end 113.03 78.74) (width 1) (layer B.Cu) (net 37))
 (segment (start 106.16 53.53) (end 106.16 55.36) (width 1) (layer B.Cu) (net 37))
 (segment (start 100.99 90.78) (end 100.99 92.71) (width 1) (layer B.Cu) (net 37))
 (segment (start 101.6 90.17) (end 100.99 90.78) (width 1) (layer B.Cu) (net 37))
 (segment (start 106.68 90.17) (end 101.6 90.17) (width 1) (layer B.Cu) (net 37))
 (segment (start 113.03 83.82) (end 106.68 90.17) (width 1) (layer B.Cu) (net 37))
 (segment (start 100.99 92.71) (end 100.33 92.71) (width 1) (layer B.Cu) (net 37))
 (segment (start 61.62 92.71) (end 61.62 87.17) (width 1) (layer B.Cu) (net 31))
 (segment (start 61.62 87.17) (end 62.23 86.56) (width 1) (layer B.Cu) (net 31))
 (segment (start 62.23 86.56) (end 62.23 78.74) (width 1) (layer B.Cu) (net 31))
 (segment (start 98.54 67.83) (end 98.54 53.53) (width 1) (layer B.Cu) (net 31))
 (segment (start 97.79 68.58) (end 98.54 67.83) (width 1) (layer B.Cu) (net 31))
 (segment (start 72.39 68.58) (end 97.79 68.58) (width 1) (layer B.Cu) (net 31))
 (segment (start 62.23 78.74) (end 72.39 68.58) (width 1) (layer B.Cu) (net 31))
 (segment (start 61.62 96.52) (end 61.62 98.45) (width 1) (layer B.Cu) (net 31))
 (segment (start 61.62 98.45) (end 62.23 99.06) (width 1) (layer B.Cu) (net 31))
 (segment (start 61.62 92.71) (end 60.96 92.71) (width 1) (layer B.Cu) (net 31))
 (segment (start 61.62 92.71) (end 61.62 96.52) (width 1) (layer B.Cu) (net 31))
 (segment (start 61.62 98.45) (end 62.23 99.06) (width 1) (layer B.Cu) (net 31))
 (segment (start 74.32 92.71) (end 74.32 87.17) (width 1) (layer B.Cu) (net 33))
 (segment (start 74.32 87.17) (end 74.93 86.56) (width 1) (layer B.Cu) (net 33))
 (segment (start 74.32 92.71) (end 73.66 92.71) (width 1) (layer B.Cu) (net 33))
 (segment (start 73.66 92.71) (end 71.12 90.17) (width 1) (layer B.Cu) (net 33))
 (segment (start 101.08 71.64) (end 101.08 53.53) (width 1) (layer B.Cu) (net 33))
 (segment (start 100.33 72.39) (end 101.08 71.64) (width 1) (layer B.Cu) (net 33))
 (segment (start 74.93 72.39) (end 100.33 72.39) (width 1) (layer B.Cu) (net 33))
 (segment (start 71.12 76.2) (end 74.93 72.39) (width 1) (layer B.Cu) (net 33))
 (segment (start 71.12 90.17) (end 71.12 76.2) (width 1) (layer B.Cu) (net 33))
 (segment (start 74.32 92.71) (end 74.32 98.45) (width 1) (layer B.Cu) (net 33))
 (segment (start 74.32 98.45) (end 74.93 99.06) (width 1) (layer B.Cu) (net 33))
 (segment (start 87.02 92.71) (end 87.02 87.17) (width 1) (layer B.Cu) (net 35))
 (segment (start 87.02 87.17) (end 87.63 86.56) (width 1) (layer B.Cu) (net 35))
 (segment (start 103.62 53.53) (end 103.62 56.63) (width 1) (layer B.Cu) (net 35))
 (segment (start 83.82 89.51) (end 87.02 92.71) (width 1) (layer B.Cu) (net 35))
 (segment (start 83.82 85.09) (end 83.82 89.51) (width 1) (layer B.Cu) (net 35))
 (segment (start 86.36 82.55) (end 83.82 85.09) (width 1) (layer B.Cu) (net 35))
 (segment (start 106.68 82.55) (end 86.36 82.55) (width 1) (layer B.Cu) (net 35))
 (segment (start 110.49 78.74) (end 106.68 82.55) (width 1) (layer B.Cu) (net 35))
 (segment (start 110.49 63.5) (end 110.49 78.74) (width 1) (layer B.Cu) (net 35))
 (segment (start 103.62 56.63) (end 110.49 63.5) (width 1) (layer B.Cu) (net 35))
 (segment (start 87.02 92.71) (end 86.36 92.71) (width 1) (layer B.Cu) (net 35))
 (segment (start 87.02 92.71) (end 87.02 98.45) (width 1) (layer B.Cu) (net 35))
 (segment (start 87.02 98.45) (end 87.63 99.06) (width 1) (layer B.Cu) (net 35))
 (segment (start 87.02 98.45) (end 87.63 99.06) (width 1) (layer B.Cu) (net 35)))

